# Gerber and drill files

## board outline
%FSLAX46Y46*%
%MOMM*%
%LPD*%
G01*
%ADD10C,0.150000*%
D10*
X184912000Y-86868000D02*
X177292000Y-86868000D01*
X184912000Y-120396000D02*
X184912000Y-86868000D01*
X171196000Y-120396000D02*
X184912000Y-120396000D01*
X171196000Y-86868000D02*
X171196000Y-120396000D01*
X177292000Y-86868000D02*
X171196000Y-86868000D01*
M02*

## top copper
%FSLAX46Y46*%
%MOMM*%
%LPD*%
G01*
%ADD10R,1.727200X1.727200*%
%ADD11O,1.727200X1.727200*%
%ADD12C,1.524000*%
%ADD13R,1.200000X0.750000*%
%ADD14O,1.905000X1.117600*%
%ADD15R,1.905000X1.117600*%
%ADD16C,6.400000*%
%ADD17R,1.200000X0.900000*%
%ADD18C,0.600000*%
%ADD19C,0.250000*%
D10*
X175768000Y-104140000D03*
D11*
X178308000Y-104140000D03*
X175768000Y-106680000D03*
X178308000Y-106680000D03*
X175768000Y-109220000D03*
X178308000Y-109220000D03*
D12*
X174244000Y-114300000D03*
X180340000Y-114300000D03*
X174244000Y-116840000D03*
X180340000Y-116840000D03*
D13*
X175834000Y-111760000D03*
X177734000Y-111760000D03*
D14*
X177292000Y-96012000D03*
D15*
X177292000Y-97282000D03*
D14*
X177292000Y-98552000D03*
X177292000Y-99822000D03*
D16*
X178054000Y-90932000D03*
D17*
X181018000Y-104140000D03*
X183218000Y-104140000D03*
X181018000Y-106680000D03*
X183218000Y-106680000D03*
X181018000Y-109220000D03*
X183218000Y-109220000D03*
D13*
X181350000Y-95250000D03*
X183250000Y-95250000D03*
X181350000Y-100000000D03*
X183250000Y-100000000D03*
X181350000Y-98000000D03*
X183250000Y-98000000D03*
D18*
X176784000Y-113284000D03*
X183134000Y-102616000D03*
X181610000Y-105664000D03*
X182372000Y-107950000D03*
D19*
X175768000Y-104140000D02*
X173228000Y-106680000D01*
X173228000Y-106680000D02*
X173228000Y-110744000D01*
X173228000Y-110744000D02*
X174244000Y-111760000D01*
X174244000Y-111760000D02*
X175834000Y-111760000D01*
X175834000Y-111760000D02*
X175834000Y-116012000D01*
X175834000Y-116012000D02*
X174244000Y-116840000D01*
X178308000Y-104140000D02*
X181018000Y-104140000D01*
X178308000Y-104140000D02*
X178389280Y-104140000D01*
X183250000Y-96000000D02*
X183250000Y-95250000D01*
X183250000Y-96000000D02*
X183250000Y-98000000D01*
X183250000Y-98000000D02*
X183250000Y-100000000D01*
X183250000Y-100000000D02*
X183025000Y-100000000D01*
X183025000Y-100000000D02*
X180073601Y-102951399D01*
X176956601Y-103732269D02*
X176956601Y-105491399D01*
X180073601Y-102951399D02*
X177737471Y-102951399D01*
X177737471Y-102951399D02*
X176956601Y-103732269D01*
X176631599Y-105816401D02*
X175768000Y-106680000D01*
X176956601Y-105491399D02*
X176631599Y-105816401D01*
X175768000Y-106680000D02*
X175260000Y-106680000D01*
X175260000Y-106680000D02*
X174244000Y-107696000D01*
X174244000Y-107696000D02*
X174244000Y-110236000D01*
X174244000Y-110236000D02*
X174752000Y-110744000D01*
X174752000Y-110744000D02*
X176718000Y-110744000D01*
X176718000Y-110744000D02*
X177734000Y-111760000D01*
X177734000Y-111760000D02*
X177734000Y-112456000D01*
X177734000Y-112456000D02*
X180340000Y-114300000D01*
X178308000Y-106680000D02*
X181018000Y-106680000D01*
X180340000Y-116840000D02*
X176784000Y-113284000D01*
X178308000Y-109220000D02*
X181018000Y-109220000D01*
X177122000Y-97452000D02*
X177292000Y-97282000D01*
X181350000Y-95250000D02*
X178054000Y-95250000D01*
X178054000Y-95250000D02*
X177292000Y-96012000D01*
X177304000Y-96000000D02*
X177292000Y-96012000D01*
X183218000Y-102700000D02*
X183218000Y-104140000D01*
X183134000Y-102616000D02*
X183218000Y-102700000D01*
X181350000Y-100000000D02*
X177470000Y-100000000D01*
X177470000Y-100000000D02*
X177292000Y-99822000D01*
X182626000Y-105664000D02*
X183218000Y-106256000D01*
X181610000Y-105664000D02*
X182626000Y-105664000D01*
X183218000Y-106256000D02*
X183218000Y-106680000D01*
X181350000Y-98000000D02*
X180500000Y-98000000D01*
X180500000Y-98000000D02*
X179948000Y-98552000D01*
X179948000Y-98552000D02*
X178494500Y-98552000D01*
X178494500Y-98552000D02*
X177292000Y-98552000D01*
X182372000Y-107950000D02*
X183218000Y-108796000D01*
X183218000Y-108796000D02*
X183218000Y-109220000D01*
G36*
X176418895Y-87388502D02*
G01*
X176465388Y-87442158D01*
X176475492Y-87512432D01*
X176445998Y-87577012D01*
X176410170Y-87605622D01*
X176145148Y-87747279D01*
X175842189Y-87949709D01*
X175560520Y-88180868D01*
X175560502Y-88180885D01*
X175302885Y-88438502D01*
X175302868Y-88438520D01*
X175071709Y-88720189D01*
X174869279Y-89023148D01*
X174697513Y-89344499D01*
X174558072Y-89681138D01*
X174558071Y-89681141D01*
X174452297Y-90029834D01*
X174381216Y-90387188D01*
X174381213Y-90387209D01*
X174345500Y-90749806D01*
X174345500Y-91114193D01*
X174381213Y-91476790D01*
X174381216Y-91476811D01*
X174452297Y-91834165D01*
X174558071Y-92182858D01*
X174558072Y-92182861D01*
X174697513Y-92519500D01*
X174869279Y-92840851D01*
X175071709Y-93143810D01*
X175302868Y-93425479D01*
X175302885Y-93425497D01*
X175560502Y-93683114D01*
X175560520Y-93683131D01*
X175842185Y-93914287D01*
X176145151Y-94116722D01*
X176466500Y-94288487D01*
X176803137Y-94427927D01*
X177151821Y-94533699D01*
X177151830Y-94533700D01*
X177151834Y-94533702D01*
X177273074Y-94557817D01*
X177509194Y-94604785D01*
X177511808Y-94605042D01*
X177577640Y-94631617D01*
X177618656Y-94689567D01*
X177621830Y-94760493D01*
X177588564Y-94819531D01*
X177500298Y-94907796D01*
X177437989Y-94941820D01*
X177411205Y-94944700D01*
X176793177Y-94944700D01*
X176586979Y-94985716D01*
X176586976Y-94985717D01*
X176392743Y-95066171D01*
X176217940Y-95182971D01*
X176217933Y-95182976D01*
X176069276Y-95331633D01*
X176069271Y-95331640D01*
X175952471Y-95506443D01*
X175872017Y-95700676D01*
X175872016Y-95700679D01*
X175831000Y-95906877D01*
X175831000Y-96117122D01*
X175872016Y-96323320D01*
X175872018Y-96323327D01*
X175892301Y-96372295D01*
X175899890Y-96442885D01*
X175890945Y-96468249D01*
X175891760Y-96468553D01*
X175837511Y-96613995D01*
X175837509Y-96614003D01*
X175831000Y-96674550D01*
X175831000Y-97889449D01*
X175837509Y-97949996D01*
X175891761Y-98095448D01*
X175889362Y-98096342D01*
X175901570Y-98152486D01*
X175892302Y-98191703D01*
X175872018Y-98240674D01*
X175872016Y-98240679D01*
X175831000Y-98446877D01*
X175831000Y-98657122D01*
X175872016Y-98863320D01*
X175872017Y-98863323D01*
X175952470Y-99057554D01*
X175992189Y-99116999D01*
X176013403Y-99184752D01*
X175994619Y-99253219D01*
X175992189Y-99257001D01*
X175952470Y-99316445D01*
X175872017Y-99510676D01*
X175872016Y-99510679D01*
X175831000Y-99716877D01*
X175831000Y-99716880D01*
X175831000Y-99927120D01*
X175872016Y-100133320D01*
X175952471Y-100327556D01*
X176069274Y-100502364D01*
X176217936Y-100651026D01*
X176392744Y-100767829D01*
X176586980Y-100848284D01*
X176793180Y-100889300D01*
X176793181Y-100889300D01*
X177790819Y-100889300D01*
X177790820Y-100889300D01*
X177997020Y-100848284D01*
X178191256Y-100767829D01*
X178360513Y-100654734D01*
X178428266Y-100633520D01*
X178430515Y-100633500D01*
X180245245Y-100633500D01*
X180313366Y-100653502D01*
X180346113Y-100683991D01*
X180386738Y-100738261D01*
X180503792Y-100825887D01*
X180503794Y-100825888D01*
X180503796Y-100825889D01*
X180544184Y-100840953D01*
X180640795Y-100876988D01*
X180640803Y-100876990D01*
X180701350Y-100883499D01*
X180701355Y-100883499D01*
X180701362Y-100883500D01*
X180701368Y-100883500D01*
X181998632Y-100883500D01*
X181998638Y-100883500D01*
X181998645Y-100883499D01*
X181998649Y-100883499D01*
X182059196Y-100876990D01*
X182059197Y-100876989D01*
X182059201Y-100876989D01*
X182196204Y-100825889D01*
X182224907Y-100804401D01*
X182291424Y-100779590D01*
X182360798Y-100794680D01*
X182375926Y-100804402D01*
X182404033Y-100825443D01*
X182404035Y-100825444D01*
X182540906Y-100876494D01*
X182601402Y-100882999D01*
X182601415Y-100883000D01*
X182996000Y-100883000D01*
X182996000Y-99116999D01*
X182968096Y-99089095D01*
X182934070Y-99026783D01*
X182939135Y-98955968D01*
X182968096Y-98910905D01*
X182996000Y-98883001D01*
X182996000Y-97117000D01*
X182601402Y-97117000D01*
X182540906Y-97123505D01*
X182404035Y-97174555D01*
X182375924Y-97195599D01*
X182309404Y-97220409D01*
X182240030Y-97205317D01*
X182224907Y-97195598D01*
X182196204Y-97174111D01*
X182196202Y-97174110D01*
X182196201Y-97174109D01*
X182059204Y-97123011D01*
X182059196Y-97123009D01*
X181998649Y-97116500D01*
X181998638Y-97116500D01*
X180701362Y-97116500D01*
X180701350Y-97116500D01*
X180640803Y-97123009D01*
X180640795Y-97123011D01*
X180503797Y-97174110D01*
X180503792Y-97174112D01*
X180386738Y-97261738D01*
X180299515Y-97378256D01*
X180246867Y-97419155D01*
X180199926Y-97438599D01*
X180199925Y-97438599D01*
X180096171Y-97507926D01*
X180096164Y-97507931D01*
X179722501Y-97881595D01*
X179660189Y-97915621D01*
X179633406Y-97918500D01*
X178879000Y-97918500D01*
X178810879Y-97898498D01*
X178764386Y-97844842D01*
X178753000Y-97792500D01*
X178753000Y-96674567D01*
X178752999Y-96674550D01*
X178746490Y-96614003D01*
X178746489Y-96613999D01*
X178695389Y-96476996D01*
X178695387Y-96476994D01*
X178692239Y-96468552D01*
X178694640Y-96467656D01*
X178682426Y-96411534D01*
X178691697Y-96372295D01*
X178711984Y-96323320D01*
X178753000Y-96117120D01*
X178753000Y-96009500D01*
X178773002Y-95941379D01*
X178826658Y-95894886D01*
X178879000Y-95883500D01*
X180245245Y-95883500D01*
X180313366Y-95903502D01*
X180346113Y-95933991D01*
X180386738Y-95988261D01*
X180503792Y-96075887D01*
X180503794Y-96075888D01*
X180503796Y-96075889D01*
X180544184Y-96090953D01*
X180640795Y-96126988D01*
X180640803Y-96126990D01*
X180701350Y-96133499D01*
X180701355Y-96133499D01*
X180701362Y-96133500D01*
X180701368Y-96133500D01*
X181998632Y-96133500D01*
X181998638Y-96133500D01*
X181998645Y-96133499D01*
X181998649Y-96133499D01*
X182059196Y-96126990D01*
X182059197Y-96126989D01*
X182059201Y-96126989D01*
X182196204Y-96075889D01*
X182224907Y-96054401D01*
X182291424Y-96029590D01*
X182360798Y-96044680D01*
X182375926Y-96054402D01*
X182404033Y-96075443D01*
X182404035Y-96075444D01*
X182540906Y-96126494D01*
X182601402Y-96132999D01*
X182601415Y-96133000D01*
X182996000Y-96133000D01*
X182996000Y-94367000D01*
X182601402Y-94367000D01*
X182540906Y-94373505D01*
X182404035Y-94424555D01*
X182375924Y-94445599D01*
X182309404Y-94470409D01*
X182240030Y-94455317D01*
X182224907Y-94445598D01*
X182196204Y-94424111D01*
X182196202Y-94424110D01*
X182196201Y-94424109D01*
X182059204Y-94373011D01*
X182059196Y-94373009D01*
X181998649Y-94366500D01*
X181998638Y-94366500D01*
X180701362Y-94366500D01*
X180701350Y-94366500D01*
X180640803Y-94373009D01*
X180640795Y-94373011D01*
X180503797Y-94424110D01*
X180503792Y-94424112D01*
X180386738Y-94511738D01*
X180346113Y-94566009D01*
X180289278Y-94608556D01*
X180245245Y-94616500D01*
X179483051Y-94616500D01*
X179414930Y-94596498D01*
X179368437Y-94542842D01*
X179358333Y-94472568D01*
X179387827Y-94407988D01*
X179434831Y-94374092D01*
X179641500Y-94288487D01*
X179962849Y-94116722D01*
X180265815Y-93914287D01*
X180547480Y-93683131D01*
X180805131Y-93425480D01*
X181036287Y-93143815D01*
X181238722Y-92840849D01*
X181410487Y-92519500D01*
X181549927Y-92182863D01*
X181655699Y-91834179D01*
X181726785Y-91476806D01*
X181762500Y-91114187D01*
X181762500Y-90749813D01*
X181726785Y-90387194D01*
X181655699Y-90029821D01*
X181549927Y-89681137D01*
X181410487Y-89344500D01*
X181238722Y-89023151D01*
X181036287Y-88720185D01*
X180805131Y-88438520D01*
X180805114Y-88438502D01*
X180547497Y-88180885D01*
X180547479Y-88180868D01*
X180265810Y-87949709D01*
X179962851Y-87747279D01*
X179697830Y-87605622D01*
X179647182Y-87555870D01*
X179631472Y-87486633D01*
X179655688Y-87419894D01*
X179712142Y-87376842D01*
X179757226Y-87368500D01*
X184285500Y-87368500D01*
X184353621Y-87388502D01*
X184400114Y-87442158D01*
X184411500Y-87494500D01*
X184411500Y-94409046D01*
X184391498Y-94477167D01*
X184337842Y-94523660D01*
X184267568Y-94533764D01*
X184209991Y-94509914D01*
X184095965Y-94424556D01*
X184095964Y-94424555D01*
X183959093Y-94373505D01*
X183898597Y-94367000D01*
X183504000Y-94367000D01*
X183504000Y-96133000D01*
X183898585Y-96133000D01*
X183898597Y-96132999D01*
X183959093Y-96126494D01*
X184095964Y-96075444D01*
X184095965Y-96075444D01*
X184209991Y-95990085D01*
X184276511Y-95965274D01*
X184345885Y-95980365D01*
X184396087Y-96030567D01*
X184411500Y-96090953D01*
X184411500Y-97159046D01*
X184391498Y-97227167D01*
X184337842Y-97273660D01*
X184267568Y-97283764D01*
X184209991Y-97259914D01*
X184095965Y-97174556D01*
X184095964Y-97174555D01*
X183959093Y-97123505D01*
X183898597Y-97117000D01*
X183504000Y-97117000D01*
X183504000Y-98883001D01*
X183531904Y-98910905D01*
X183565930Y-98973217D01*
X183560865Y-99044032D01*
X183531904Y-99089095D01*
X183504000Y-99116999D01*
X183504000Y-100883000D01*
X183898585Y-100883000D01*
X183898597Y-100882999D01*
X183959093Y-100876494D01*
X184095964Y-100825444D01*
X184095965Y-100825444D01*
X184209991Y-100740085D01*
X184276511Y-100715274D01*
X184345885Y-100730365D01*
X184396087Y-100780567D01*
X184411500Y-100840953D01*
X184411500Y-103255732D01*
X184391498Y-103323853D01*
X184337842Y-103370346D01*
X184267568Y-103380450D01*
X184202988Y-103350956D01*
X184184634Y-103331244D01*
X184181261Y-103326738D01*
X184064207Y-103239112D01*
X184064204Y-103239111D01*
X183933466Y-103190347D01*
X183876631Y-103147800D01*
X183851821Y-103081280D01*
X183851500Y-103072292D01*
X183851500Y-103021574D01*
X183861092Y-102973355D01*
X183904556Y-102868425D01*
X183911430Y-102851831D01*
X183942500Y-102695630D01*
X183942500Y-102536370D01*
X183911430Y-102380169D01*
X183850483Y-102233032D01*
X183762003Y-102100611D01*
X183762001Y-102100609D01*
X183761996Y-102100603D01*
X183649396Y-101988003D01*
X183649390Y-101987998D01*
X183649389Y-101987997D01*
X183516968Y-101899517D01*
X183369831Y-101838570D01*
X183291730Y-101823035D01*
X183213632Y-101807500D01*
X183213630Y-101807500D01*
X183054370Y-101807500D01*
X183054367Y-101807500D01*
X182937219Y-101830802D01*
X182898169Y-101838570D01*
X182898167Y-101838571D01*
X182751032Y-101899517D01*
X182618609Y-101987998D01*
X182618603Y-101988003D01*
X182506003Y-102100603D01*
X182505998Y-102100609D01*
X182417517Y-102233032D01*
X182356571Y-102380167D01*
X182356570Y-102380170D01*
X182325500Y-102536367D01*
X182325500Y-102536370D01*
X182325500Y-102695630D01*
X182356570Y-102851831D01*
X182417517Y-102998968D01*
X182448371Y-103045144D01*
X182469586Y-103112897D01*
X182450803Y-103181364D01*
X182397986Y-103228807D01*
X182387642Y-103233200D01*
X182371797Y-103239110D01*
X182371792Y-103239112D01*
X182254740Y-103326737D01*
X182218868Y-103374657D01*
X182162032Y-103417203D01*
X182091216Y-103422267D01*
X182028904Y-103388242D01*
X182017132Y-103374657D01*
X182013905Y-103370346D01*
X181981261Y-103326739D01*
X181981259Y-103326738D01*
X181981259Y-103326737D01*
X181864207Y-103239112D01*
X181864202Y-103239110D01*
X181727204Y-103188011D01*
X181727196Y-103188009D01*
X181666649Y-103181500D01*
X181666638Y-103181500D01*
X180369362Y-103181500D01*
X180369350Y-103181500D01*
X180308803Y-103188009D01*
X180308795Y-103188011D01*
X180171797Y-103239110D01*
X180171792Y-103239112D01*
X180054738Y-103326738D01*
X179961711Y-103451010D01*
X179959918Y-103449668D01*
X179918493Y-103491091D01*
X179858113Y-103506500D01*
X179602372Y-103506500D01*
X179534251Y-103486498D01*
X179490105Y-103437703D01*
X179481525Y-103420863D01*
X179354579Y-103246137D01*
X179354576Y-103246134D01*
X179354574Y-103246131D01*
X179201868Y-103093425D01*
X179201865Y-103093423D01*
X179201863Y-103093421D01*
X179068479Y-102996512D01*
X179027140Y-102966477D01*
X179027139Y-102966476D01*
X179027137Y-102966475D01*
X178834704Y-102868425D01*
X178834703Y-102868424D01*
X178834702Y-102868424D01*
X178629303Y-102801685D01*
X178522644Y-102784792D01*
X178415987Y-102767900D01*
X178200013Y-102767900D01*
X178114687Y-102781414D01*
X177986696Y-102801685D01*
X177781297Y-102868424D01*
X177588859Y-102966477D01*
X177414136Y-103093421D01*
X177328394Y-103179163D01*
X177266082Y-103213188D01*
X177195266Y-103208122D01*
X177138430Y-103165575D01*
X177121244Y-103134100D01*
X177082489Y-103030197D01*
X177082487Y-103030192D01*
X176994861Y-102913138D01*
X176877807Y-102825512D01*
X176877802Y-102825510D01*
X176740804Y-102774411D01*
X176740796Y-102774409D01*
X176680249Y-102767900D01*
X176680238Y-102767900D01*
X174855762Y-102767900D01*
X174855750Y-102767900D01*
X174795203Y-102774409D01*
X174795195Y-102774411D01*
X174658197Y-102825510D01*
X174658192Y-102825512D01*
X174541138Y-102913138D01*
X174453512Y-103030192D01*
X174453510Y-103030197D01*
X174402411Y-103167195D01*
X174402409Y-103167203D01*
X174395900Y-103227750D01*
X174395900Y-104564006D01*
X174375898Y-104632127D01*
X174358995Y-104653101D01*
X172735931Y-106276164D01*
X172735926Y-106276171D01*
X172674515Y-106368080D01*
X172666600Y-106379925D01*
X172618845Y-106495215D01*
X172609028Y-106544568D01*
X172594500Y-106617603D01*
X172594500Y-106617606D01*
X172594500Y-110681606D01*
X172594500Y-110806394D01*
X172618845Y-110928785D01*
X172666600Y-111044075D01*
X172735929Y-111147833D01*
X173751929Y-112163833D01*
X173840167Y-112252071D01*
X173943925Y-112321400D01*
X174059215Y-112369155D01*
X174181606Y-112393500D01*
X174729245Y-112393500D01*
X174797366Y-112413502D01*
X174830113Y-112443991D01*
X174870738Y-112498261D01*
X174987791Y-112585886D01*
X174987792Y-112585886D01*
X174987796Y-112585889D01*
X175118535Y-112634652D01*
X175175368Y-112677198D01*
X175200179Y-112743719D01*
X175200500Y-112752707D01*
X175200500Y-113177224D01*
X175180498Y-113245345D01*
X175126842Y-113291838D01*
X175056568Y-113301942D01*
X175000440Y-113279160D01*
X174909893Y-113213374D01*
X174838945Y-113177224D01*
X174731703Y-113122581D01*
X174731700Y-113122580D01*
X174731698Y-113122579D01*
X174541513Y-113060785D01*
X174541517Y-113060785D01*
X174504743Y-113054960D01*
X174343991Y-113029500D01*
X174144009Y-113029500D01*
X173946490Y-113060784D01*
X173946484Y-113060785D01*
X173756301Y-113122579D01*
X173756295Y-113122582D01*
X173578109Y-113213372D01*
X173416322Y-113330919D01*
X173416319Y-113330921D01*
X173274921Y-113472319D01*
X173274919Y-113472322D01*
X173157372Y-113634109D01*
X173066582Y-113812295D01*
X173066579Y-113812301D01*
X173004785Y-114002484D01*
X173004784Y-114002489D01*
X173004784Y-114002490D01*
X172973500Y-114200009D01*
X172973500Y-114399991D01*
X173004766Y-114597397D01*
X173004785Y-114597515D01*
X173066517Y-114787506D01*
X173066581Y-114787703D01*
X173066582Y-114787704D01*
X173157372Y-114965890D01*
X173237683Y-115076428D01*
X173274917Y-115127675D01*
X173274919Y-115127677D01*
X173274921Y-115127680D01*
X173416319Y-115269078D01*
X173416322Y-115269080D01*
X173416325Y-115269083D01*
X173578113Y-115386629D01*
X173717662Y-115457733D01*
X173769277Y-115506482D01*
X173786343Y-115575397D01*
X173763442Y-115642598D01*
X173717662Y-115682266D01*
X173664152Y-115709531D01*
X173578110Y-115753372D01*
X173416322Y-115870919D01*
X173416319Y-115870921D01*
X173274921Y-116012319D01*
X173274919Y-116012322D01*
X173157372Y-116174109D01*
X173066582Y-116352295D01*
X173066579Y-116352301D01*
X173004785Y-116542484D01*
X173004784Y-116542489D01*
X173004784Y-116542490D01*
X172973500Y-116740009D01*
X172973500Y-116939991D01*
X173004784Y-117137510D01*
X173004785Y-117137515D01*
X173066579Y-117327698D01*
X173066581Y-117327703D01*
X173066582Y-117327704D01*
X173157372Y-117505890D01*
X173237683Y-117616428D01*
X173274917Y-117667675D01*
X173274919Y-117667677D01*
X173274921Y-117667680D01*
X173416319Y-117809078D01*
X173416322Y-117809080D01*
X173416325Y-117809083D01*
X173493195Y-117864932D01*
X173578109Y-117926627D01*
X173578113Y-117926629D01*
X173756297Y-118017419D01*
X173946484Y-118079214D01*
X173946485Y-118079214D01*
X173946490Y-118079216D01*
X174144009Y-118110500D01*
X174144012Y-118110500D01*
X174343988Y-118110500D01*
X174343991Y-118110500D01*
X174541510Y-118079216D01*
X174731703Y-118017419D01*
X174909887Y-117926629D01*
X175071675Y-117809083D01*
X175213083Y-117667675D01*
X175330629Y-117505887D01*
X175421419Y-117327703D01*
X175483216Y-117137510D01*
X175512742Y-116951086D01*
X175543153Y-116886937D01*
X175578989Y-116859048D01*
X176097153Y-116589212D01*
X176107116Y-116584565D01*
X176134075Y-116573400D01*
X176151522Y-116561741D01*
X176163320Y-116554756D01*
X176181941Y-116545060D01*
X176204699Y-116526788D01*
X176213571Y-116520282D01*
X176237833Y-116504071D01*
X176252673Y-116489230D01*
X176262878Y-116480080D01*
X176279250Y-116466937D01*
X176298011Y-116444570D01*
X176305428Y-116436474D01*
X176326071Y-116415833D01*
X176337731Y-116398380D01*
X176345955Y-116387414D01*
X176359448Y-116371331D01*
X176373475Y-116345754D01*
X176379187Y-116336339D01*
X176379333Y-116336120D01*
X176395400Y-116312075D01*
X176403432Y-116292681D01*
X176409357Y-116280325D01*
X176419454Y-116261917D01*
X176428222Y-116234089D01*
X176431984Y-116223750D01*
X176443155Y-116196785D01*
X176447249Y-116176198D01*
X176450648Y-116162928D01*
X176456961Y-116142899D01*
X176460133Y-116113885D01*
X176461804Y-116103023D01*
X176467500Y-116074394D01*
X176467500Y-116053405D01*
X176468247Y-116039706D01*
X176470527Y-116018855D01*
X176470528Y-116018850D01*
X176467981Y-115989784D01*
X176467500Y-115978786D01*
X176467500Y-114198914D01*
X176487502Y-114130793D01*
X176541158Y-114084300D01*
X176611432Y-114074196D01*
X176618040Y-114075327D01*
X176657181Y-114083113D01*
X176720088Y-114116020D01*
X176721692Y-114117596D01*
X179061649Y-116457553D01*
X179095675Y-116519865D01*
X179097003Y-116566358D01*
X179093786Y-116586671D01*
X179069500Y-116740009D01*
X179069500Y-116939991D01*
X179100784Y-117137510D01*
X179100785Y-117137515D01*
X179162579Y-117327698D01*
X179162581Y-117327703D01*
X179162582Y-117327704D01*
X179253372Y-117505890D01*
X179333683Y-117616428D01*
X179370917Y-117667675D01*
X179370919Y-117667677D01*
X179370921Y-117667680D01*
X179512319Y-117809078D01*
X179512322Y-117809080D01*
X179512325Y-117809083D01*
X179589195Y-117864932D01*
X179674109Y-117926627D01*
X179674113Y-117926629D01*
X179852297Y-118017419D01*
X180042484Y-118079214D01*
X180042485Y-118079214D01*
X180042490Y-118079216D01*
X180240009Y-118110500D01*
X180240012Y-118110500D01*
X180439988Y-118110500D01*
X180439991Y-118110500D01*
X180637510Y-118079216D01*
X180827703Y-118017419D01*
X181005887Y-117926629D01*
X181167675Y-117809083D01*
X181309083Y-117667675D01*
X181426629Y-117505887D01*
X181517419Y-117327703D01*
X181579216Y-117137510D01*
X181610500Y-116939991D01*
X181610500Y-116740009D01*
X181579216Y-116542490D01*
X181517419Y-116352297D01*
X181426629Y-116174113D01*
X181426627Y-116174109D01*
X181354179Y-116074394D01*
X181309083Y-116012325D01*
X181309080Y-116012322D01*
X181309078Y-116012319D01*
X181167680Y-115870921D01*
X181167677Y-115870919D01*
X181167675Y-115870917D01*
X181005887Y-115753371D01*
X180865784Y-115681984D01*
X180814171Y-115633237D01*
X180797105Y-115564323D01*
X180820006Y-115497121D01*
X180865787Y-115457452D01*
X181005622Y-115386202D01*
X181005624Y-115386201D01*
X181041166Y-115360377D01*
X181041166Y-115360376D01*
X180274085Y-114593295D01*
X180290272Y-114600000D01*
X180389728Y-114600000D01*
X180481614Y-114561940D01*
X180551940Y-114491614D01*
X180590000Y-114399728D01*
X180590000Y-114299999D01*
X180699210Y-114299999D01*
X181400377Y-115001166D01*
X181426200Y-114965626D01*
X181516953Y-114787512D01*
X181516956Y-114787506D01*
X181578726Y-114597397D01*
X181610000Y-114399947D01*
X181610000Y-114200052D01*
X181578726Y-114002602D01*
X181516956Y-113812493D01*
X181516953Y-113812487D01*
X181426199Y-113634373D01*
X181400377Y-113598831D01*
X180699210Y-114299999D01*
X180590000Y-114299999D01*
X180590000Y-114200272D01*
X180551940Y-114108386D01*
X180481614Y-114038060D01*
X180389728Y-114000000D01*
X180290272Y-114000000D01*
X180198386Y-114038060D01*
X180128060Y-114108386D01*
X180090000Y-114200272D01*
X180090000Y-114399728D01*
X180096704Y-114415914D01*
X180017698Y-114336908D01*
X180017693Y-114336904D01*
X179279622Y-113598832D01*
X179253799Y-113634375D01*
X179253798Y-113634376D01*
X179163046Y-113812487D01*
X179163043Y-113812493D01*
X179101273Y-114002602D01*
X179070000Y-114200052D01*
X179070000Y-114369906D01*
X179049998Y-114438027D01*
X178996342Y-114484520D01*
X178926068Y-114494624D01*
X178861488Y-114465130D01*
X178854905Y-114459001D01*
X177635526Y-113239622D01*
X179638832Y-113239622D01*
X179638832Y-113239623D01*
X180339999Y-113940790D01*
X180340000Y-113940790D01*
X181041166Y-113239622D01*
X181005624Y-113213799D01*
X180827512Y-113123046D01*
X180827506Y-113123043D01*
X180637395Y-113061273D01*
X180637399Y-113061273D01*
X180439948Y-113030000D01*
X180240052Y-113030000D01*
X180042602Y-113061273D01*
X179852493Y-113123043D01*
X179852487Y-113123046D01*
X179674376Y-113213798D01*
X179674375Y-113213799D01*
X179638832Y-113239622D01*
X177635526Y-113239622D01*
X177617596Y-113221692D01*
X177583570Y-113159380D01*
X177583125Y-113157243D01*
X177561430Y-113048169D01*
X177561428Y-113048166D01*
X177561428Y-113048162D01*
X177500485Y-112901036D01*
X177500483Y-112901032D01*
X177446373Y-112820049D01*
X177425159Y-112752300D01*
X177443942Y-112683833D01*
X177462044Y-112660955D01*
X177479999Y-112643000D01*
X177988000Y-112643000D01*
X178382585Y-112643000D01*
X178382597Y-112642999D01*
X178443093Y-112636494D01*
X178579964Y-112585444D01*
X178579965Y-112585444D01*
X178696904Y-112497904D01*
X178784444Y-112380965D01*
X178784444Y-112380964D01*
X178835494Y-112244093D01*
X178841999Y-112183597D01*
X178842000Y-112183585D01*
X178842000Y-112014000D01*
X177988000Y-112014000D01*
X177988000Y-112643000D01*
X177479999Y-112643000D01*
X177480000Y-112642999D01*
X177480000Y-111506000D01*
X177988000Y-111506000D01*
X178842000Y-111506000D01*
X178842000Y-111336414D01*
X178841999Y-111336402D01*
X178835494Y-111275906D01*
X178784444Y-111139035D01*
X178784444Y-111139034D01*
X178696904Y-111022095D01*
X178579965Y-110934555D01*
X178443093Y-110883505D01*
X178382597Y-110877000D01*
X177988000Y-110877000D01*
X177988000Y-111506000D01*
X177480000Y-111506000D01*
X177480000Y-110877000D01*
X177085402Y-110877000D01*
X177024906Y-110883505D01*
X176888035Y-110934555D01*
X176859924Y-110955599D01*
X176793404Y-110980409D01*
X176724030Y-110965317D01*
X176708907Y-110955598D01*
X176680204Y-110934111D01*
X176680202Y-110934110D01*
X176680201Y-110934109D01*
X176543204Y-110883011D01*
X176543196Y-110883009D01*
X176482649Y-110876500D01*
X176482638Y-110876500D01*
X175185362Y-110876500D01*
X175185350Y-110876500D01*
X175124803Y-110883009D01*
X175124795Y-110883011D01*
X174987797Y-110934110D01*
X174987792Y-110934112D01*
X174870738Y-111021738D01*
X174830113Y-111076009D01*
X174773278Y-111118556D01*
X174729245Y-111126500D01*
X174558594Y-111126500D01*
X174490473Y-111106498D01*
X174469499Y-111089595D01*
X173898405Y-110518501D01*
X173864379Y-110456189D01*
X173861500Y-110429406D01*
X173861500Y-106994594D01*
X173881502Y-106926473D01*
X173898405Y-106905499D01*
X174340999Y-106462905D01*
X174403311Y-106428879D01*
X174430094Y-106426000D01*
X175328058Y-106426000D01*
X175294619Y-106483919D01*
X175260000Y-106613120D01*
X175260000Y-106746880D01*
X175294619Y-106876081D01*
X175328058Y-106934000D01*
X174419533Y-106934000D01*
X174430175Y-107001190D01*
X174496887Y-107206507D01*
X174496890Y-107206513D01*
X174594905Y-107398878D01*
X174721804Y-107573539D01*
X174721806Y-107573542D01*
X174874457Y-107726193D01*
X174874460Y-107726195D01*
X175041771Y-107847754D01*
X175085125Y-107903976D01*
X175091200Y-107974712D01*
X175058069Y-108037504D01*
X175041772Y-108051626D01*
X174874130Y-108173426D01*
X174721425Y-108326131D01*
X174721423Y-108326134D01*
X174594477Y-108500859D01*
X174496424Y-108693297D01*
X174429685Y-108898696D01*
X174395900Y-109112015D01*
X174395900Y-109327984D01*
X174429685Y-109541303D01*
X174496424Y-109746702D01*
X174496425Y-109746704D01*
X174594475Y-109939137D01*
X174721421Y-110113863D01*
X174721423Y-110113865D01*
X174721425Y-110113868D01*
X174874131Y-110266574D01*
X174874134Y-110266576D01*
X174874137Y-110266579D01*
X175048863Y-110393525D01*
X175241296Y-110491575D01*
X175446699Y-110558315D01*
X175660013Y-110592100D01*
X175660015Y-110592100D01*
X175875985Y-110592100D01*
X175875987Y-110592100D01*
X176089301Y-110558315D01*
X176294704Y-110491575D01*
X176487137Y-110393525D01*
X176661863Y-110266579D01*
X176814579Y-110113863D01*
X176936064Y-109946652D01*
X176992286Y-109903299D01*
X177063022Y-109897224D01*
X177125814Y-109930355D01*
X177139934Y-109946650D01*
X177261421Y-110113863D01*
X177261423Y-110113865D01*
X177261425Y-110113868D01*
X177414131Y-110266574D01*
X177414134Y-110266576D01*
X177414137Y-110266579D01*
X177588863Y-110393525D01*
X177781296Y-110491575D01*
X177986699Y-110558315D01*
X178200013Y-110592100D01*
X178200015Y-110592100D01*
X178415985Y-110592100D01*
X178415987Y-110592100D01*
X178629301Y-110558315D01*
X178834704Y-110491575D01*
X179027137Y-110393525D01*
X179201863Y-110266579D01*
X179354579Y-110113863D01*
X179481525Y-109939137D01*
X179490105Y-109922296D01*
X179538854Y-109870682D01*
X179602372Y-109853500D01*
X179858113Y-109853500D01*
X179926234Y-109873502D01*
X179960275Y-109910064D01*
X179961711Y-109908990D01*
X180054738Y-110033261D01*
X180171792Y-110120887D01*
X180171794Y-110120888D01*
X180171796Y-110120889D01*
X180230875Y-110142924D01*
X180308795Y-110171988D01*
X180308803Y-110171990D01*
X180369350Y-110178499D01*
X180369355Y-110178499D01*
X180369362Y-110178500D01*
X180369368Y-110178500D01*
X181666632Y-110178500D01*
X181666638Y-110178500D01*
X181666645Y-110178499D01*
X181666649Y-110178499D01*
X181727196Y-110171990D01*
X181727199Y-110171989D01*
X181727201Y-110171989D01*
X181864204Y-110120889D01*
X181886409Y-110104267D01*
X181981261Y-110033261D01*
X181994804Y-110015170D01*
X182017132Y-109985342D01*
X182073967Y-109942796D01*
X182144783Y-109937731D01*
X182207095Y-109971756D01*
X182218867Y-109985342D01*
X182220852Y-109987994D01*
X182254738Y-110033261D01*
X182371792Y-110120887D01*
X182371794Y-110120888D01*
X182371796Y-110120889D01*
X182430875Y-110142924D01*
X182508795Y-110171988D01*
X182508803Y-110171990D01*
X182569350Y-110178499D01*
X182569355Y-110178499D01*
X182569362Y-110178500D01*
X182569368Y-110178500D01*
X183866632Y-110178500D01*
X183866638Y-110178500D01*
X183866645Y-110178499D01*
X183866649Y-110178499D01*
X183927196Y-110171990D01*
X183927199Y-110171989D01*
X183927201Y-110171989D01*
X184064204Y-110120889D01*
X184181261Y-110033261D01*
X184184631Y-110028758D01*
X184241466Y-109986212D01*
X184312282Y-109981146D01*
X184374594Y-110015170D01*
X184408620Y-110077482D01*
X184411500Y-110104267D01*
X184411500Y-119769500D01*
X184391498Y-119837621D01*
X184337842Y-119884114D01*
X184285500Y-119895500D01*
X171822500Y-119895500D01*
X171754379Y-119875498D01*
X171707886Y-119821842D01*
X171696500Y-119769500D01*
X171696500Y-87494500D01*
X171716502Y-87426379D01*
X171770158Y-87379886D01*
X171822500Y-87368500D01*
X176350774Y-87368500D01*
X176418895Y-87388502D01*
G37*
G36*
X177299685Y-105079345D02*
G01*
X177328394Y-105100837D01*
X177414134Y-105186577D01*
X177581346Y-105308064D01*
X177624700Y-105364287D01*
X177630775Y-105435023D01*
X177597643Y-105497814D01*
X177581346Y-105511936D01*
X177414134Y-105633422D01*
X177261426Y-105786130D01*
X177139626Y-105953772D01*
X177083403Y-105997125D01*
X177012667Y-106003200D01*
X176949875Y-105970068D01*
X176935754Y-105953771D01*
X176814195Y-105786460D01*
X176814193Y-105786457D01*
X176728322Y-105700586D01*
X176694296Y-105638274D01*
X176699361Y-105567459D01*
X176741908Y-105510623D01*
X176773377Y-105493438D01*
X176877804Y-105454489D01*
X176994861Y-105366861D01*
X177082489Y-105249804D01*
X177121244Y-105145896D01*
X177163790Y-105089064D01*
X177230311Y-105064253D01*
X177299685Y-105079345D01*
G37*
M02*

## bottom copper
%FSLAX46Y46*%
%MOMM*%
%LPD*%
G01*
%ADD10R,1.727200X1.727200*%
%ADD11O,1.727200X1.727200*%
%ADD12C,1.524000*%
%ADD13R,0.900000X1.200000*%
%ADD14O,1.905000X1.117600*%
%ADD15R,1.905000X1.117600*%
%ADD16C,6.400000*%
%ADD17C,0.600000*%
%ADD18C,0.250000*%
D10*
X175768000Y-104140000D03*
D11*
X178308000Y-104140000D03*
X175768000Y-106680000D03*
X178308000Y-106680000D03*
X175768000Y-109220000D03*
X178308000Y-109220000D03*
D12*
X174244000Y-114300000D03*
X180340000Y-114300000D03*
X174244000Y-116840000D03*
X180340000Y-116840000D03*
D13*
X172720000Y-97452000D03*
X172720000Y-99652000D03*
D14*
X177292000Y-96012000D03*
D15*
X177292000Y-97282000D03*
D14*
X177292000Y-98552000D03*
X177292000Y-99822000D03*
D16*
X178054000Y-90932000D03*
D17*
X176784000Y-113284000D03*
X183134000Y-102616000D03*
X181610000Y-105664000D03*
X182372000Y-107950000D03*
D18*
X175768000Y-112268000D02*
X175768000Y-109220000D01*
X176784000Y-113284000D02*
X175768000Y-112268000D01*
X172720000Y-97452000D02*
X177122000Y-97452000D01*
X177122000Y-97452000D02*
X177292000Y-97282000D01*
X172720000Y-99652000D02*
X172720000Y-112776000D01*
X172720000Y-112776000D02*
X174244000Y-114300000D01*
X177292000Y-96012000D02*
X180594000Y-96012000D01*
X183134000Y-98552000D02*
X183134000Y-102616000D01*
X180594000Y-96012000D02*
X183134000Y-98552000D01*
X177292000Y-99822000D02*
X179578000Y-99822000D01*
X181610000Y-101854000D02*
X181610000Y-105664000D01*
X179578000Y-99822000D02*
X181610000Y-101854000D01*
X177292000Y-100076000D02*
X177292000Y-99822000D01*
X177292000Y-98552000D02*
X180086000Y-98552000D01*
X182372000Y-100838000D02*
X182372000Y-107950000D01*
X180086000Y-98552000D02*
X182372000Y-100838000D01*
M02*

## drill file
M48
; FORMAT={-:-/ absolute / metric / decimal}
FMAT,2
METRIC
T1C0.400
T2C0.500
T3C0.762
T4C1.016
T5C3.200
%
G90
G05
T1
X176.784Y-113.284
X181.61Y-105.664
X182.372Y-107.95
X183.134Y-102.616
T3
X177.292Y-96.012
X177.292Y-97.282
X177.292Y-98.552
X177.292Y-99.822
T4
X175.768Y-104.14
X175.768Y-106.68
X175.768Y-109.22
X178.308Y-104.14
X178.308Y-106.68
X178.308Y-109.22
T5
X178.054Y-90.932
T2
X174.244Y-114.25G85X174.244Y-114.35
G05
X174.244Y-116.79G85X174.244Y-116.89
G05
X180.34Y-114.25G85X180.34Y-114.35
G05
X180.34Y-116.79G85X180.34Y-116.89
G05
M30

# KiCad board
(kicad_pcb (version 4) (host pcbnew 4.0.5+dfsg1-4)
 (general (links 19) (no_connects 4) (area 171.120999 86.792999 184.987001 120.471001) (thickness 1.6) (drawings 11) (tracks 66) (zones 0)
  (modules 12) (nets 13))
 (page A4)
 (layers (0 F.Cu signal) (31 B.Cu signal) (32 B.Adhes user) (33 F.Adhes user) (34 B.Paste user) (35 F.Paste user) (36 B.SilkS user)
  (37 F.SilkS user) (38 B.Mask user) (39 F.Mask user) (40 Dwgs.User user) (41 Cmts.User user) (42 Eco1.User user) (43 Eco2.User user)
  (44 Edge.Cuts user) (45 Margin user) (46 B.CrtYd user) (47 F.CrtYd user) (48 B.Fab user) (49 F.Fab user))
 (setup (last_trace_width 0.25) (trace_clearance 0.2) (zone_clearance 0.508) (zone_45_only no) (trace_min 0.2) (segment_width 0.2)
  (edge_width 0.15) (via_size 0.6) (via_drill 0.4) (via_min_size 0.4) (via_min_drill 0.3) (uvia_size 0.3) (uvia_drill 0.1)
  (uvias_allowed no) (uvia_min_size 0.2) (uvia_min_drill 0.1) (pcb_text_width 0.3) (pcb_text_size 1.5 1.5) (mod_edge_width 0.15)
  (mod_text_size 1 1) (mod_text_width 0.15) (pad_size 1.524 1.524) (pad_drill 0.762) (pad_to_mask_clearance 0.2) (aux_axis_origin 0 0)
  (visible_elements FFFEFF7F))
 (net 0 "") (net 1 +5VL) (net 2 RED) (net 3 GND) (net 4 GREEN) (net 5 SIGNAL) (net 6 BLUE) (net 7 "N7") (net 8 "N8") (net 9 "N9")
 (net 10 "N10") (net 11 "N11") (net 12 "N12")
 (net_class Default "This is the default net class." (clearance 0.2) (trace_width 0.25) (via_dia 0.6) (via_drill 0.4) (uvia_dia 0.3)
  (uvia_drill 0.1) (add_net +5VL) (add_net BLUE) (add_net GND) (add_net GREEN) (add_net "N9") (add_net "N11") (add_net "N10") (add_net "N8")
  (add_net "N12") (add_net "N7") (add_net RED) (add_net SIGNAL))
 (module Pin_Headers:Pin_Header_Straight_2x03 (layer F.Cu) (at 175.768 104.14)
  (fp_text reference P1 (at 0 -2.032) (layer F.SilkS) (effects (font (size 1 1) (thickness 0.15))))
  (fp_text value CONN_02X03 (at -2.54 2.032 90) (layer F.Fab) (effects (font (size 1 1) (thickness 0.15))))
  (pad 1 thru_hole rect (at 0 0) (size 1.7272 1.7272) (drill 1.016) (layers *.Cu *.Mask) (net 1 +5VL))
  (pad 2 thru_hole oval (at 2.54 0) (size 1.7272 1.7272) (drill 1.016) (layers *.Cu *.Mask) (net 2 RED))
  (pad 3 thru_hole oval (at 0 2.54) (size 1.7272 1.7272) (drill 1.016) (layers *.Cu *.Mask) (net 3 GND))
  (pad 4 thru_hole oval (at 2.54 2.54) (size 1.7272 1.7272) (drill 1.016) (layers *.Cu *.Mask) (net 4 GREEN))
  (pad 5 thru_hole oval (at 0 5.08) (size 1.7272 1.7272) (drill 1.016) (layers *.Cu *.Mask) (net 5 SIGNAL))
  (pad 6 thru_hole oval (at 2.54 5.08) (size 1.7272 1.7272) (drill 1.016) (layers *.Cu *.Mask) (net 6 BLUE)))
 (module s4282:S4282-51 (layer F.Cu) (at 177.292 115.57)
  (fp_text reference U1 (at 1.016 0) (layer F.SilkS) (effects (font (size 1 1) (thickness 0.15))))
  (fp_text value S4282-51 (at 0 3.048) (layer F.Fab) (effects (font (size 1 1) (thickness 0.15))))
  (pad 1 thru_hole circle (at -3.048 -1.27) (size 1.524 1.524) (drill oval 0.5 0.6) (layers *.Cu *.Mask F.SilkS) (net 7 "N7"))
  (pad 4 thru_hole circle (at 3.048 -1.27) (size 1.524 1.524) (drill oval 0.5 0.6) (layers *.Cu *.Mask F.SilkS) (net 3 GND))
  (pad 2 thru_hole circle (at -3.048 1.27) (size 1.524 1.524) (drill oval 0.5 0.6) (layers *.Cu *.Mask F.SilkS) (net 1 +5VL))
  (pad 3 thru_hole circle (at 3.048 1.27) (size 1.524 1.524) (drill oval 0.5 0.6) (layers *.Cu *.Mask F.SilkS) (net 5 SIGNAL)))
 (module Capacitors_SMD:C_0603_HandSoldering (layer F.Cu) (at 176.784 111.76)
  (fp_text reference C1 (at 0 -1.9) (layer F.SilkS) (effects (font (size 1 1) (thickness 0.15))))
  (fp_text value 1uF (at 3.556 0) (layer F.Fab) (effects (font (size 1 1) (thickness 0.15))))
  (pad 1 smd rect (at -0.95 0) (size 1.2 0.75) (layers F.Cu F.Paste F.Mask) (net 1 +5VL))
  (pad 2 smd rect (at 0.95 0) (size 1.2 0.75) (layers F.Cu F.Paste F.Mask) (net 3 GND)))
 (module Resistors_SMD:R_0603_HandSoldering (layer B.Cu) (at 172.72 98.552 270)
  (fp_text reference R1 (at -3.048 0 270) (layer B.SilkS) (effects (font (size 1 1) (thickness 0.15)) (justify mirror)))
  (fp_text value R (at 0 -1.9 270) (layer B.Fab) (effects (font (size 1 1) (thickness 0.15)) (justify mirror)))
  (pad 1 smd rect (at -1.1 0 270) (size 1.2 0.9) (layers B.Cu B.Paste B.Mask) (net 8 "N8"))
  (pad 2 smd rect (at 1.1 0 270) (size 1.2 0.9) (layers B.Cu B.Paste B.Mask) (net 7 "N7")))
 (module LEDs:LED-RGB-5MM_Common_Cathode (layer F.Cu) (at 177.292 96.012)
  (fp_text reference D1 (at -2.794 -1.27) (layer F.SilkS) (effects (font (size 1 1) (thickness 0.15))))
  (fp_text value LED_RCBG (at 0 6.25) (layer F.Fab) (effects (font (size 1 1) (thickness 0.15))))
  (pad 1 thru_hole oval (at 0 0) (size 1.905 1.1176) (drill 0.762) (layers *.Cu *.Mask) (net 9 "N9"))
  (pad 2 thru_hole rect (at 0 1.27) (size 1.905 1.1176) (drill 0.762) (layers *.Cu *.Mask) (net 8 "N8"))
  (pad 3 thru_hole oval (at 0 2.54) (size 1.905 1.1176) (drill 0.762) (layers *.Cu *.Mask) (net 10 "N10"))
  (pad 4 thru_hole oval (at 0 3.81) (size 1.905 1.1176) (drill 0.762) (layers *.Cu *.Mask) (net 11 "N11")))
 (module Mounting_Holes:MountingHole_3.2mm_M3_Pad (layer F.Cu) (at 178.054 90.932)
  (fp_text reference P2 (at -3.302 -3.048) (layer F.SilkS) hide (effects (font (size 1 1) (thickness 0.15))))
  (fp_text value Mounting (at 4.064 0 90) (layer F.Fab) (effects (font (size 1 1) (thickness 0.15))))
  (pad 1 thru_hole circle (at 0 0) (size 6.4 6.4) (drill 3.2) (layers *.Cu *.Mask) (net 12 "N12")))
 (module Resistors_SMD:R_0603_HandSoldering (layer F.Cu) (at 182.118 104.14)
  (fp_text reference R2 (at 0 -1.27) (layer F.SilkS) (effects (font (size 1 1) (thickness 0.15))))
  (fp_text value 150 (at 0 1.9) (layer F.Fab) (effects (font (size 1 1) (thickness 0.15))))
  (pad 1 smd rect (at -1.1 0) (size 1.2 0.9) (layers F.Cu F.Paste F.Mask) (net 2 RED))
  (pad 2 smd rect (at 1.1 0) (size 1.2 0.9) (layers F.Cu F.Paste F.Mask) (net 9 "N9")))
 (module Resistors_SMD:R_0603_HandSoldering (layer F.Cu) (at 182.118 106.68)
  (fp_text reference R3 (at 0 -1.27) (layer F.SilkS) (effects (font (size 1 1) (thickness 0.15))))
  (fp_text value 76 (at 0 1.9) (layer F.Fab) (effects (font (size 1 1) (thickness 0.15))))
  (pad 1 smd rect (at -1.1 0) (size 1.2 0.9) (layers F.Cu F.Paste F.Mask) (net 4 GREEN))
  (pad 2 smd rect (at 1.1 0) (size 1.2 0.9) (layers F.Cu F.Paste F.Mask) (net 11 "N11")))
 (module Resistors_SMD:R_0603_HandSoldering (layer F.Cu) (at 182.118 109.22)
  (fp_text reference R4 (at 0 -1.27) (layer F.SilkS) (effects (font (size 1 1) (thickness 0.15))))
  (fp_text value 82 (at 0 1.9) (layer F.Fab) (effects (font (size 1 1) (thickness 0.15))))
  (pad 1 smd rect (at -1.1 0) (size 1.2 0.9) (layers F.Cu F.Paste F.Mask) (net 6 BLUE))
  (pad 2 smd rect (at 1.1 0) (size 1.2 0.9) (layers F.Cu F.Paste F.Mask) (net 10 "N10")))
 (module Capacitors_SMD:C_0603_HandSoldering (layer F.Cu) (at 182.3 95.25)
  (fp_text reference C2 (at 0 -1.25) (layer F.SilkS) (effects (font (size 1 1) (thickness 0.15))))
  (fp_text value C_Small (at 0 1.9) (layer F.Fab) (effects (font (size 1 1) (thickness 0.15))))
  (pad 1 smd rect (at -0.95 0) (size 1.2 0.75) (layers F.Cu F.Paste F.Mask) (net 9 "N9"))
  (pad 2 smd rect (at 0.95 0) (size 1.2 0.75) (layers F.Cu F.Paste F.Mask) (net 3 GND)))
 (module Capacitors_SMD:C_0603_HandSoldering (layer F.Cu) (at 182.3 100)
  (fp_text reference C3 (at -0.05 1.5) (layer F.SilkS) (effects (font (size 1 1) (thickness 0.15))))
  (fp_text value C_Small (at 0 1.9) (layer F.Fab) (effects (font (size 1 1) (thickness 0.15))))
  (pad 1 smd rect (at -0.95 0) (size 1.2 0.75) (layers F.Cu F.Paste F.Mask) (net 11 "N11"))
  (pad 2 smd rect (at 0.95 0) (size 1.2 0.75) (layers F.Cu F.Paste F.Mask) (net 3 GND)))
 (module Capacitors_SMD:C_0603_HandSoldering (layer F.Cu) (at 182.3 98)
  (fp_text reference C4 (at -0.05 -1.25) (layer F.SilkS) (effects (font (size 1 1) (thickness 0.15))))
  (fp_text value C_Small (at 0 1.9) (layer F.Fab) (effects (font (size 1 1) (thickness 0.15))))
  (pad 1 smd rect (at -0.95 0) (size 1.2 0.75) (layers F.Cu F.Paste F.Mask) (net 10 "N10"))
  (pad 2 smd rect (at 0.95 0) (size 1.2 0.75) (layers F.Cu F.Paste F.Mask) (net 3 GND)))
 (gr_line (start 184.912 86.868) (end 177.292 86.868) (angle 90) (layer Edge.Cuts) (width 0.15))
 (gr_line (start 184.912 120.396) (end 184.912 86.868) (angle 90) (layer Edge.Cuts) (width 0.15))
 (gr_line (start 171.196 120.396) (end 184.912 120.396) (angle 90) (layer Edge.Cuts) (width 0.15))
 (gr_line (start 171.196 86.868) (end 171.196 120.396) (angle 90) (layer Edge.Cuts) (width 0.15))
 (gr_line (start 177.292 86.868) (end 171.196 86.868) (angle 90) (layer Edge.Cuts) (width 0.15))
 (segment (start 175.768 104.14) (end 173.228 106.68) (width 0.25) (layer F.Cu) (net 1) (status 10))
 (segment (start 173.228 106.68) (end 173.228 110.744) (width 0.25) (layer F.Cu) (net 1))
 (segment (start 173.228 110.744) (end 174.244 111.76) (width 0.25) (layer F.Cu) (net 1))
 (segment (start 174.244 111.76) (end 175.834 111.76) (width 0.25) (layer F.Cu) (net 1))
 (segment (start 175.834 111.76) (end 175.834 116.012) (width 0.25) (layer F.Cu) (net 1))
 (segment (start 175.834 116.012) (end 174.244 116.84) (width 0.25) (layer F.Cu) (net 1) (status 20))
 (segment (start 178.308 104.14) (end 181.018 104.14) (width 0.25) (layer F.Cu) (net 2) (status 10))
 (segment (start 178.308 104.14) (end 178.38928 104.14) (width 0.25) (layer F.Cu) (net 2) (status 30))
 (segment (start 183.25 96) (end 183.25 95.25) (width 0.25) (layer F.Cu) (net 3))
 (segment (start 183.25 96) (end 183.25 98) (width 0.25) (layer F.Cu) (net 3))
 (segment (start 183.25 98) (end 183.25 100) (width 0.25) (layer F.Cu) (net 3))
 (segment (start 183.25 100) (end 183.025 100) (width 0.25) (layer F.Cu) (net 3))
 (segment (start 183.025 100) (end 180.073601 102.951399) (width 0.25) (layer F.Cu) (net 3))
 (segment (start 176.956601 103.732269) (end 176.956601 105.491399) (width 0.25) (layer F.Cu) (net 3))
 (segment (start 180.073601 102.951399) (end 177.737471 102.951399) (width 0.25) (layer F.Cu) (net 3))
 (segment (start 177.737471 102.951399) (end 176.956601 103.732269) (width 0.25) (layer F.Cu) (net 3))
 (segment (start 176.631599 105.816401) (end 175.768 106.68) (width 0.25) (layer F.Cu) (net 3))
 (segment (start 176.956601 105.491399) (end 176.631599 105.816401) (width 0.25) (layer F.Cu) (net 3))
 (segment (start 175.768 106.68) (end 175.26 106.68) (width 0.25) (layer F.Cu) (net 3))
 (segment (start 175.26 106.68) (end 174.244 107.696) (width 0.25) (layer F.Cu) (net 3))
 (segment (start 174.244 107.696) (end 174.244 110.236) (width 0.25) (layer F.Cu) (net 3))
 (segment (start 174.244 110.236) (end 174.752 110.744) (width 0.25) (layer F.Cu) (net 3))
 (segment (start 174.752 110.744) (end 176.718 110.744) (width 0.25) (layer F.Cu) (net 3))
 (segment (start 176.718 110.744) (end 177.734 111.76) (width 0.25) (layer F.Cu) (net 3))
 (segment (start 177.734 111.76) (end 177.734 112.456) (width 0.25) (layer F.Cu) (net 3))
 (segment (start 177.734 112.456) (end 180.34 114.3) (width 0.25) (layer F.Cu) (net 3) (status 20))
 (segment (start 178.308 106.68) (end 181.018 106.68) (width 0.25) (layer F.Cu) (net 4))
 (segment (start 180.34 116.84) (end 176.784 113.284) (width 0.25) (layer F.Cu) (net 5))
 (segment (start 175.768 112.268) (end 175.768 109.22) (width 0.25) (layer B.Cu) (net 5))
 (segment (start 176.784 113.284) (end 175.768 112.268) (width 0.25) (layer B.Cu) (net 5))
 (via (at 176.784 113.284) (size 0.6) (drill 0.4) (layers F.Cu B.Cu) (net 5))
 (segment (start 178.308 109.22) (end 181.018 109.22) (width 0.25) (layer F.Cu) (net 6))
 (segment (start 172.72 97.452) (end 177.122 97.452) (width 0.25) (layer B.Cu) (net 8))
 (segment (start 177.122 97.452) (end 177.292 97.282) (width 0.25) (layer B.Cu) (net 8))
 (segment (start 177.122 97.452) (end 177.292 97.282) (width 0.25) (layer F.Cu) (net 8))
 (segment (start 172.72 99.652) (end 172.72 112.776) (width 0.25) (layer B.Cu) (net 7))
 (segment (start 172.72 112.776) (end 174.244 114.3) (width 0.25) (layer B.Cu) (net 7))
 (segment (start 181.35 95.25) (end 178.054 95.25) (width 0.25) (layer F.Cu) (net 9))
 (segment (start 178.054 95.25) (end 177.292 96.012) (width 0.25) (layer F.Cu) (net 9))
 (segment (start 177.304 96) (end 177.292 96.012) (width 0.25) (layer F.Cu) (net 9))
 (segment (start 177.292 96.012) (end 180.594 96.012) (width 0.25) (layer B.Cu) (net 9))
 (segment (start 183.218 102.7) (end 183.218 104.14) (width 0.25) (layer F.Cu) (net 9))
 (segment (start 183.134 102.616) (end 183.218 102.7) (width 0.25) (layer F.Cu) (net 9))
 (via (at 183.134 102.616) (size 0.6) (drill 0.4) (layers F.Cu B.Cu) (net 9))
 (segment (start 183.134 98.552) (end 183.134 102.616) (width 0.25) (layer B.Cu) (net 9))
 (segment (start 180.594 96.012) (end 183.134 98.552) (width 0.25) (layer B.Cu) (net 9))
 (segment (start 181.35 100) (end 177.47 100) (width 0.25) (layer F.Cu) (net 11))
 (segment (start 177.47 100) (end 177.292 99.822) (width 0.25) (layer F.Cu) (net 11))
 (segment (start 177.292 99.822) (end 179.578 99.822) (width 0.25) (layer B.Cu) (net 11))
 (segment (start 182.626 105.664) (end 183.218 106.256) (width 0.25) (layer F.Cu) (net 11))
 (segment (start 181.61 105.664) (end 182.626 105.664) (width 0.25) (layer F.Cu) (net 11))
 (via (at 181.61 105.664) (size 0.6) (drill 0.4) (layers F.Cu B.Cu) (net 11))
 (segment (start 181.61 101.854) (end 181.61 105.664) (width 0.25) (layer B.Cu) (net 11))
 (segment (start 179.578 99.822) (end 181.61 101.854) (width 0.25) (layer B.Cu) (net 11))
 (segment (start 183.218 106.256) (end 183.218 106.68) (width 0.25) (layer F.Cu) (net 11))
 (segment (start 177.292 100.076) (end 177.292 99.822) (width 0.25) (layer B.Cu) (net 11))
 (segment (start 181.35 98) (end 180.5 98) (width 0.25) (layer F.Cu) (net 10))
 (segment (start 180.5 98) (end 179.948 98.552) (width 0.25) (layer F.Cu) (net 10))
 (segment (start 179.948 98.552) (end 178.4945 98.552) (width 0.25) (layer F.Cu) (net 10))
 (segment (start 178.4945 98.552) (end 177.292 98.552) (width 0.25) (layer F.Cu) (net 10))
 (segment (start 177.292 98.552) (end 180.086 98.552) (width 0.25) (layer B.Cu) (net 10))
 (segment (start 182.372 107.95) (end 183.218 108.796) (width 0.25) (layer F.Cu) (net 10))
 (via (at 182.372 107.95) (size 0.6) (drill 0.4) (layers F.Cu B.Cu) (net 10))
 (segment (start 182.372 100.838) (end 182.372 107.95) (width 0.25) (layer B.Cu) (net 10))
 (segment (start 180.086 98.552) (end 182.372 100.838) (width 0.25) (layer B.Cu) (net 10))
 (segment (start 183.218 108.796) (end 183.218 109.22) (width 0.25) (layer F.Cu) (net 10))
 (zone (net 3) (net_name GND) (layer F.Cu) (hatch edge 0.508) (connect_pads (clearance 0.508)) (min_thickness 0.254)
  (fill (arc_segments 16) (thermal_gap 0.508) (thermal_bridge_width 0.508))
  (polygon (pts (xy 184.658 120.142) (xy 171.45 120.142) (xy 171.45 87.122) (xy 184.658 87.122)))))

